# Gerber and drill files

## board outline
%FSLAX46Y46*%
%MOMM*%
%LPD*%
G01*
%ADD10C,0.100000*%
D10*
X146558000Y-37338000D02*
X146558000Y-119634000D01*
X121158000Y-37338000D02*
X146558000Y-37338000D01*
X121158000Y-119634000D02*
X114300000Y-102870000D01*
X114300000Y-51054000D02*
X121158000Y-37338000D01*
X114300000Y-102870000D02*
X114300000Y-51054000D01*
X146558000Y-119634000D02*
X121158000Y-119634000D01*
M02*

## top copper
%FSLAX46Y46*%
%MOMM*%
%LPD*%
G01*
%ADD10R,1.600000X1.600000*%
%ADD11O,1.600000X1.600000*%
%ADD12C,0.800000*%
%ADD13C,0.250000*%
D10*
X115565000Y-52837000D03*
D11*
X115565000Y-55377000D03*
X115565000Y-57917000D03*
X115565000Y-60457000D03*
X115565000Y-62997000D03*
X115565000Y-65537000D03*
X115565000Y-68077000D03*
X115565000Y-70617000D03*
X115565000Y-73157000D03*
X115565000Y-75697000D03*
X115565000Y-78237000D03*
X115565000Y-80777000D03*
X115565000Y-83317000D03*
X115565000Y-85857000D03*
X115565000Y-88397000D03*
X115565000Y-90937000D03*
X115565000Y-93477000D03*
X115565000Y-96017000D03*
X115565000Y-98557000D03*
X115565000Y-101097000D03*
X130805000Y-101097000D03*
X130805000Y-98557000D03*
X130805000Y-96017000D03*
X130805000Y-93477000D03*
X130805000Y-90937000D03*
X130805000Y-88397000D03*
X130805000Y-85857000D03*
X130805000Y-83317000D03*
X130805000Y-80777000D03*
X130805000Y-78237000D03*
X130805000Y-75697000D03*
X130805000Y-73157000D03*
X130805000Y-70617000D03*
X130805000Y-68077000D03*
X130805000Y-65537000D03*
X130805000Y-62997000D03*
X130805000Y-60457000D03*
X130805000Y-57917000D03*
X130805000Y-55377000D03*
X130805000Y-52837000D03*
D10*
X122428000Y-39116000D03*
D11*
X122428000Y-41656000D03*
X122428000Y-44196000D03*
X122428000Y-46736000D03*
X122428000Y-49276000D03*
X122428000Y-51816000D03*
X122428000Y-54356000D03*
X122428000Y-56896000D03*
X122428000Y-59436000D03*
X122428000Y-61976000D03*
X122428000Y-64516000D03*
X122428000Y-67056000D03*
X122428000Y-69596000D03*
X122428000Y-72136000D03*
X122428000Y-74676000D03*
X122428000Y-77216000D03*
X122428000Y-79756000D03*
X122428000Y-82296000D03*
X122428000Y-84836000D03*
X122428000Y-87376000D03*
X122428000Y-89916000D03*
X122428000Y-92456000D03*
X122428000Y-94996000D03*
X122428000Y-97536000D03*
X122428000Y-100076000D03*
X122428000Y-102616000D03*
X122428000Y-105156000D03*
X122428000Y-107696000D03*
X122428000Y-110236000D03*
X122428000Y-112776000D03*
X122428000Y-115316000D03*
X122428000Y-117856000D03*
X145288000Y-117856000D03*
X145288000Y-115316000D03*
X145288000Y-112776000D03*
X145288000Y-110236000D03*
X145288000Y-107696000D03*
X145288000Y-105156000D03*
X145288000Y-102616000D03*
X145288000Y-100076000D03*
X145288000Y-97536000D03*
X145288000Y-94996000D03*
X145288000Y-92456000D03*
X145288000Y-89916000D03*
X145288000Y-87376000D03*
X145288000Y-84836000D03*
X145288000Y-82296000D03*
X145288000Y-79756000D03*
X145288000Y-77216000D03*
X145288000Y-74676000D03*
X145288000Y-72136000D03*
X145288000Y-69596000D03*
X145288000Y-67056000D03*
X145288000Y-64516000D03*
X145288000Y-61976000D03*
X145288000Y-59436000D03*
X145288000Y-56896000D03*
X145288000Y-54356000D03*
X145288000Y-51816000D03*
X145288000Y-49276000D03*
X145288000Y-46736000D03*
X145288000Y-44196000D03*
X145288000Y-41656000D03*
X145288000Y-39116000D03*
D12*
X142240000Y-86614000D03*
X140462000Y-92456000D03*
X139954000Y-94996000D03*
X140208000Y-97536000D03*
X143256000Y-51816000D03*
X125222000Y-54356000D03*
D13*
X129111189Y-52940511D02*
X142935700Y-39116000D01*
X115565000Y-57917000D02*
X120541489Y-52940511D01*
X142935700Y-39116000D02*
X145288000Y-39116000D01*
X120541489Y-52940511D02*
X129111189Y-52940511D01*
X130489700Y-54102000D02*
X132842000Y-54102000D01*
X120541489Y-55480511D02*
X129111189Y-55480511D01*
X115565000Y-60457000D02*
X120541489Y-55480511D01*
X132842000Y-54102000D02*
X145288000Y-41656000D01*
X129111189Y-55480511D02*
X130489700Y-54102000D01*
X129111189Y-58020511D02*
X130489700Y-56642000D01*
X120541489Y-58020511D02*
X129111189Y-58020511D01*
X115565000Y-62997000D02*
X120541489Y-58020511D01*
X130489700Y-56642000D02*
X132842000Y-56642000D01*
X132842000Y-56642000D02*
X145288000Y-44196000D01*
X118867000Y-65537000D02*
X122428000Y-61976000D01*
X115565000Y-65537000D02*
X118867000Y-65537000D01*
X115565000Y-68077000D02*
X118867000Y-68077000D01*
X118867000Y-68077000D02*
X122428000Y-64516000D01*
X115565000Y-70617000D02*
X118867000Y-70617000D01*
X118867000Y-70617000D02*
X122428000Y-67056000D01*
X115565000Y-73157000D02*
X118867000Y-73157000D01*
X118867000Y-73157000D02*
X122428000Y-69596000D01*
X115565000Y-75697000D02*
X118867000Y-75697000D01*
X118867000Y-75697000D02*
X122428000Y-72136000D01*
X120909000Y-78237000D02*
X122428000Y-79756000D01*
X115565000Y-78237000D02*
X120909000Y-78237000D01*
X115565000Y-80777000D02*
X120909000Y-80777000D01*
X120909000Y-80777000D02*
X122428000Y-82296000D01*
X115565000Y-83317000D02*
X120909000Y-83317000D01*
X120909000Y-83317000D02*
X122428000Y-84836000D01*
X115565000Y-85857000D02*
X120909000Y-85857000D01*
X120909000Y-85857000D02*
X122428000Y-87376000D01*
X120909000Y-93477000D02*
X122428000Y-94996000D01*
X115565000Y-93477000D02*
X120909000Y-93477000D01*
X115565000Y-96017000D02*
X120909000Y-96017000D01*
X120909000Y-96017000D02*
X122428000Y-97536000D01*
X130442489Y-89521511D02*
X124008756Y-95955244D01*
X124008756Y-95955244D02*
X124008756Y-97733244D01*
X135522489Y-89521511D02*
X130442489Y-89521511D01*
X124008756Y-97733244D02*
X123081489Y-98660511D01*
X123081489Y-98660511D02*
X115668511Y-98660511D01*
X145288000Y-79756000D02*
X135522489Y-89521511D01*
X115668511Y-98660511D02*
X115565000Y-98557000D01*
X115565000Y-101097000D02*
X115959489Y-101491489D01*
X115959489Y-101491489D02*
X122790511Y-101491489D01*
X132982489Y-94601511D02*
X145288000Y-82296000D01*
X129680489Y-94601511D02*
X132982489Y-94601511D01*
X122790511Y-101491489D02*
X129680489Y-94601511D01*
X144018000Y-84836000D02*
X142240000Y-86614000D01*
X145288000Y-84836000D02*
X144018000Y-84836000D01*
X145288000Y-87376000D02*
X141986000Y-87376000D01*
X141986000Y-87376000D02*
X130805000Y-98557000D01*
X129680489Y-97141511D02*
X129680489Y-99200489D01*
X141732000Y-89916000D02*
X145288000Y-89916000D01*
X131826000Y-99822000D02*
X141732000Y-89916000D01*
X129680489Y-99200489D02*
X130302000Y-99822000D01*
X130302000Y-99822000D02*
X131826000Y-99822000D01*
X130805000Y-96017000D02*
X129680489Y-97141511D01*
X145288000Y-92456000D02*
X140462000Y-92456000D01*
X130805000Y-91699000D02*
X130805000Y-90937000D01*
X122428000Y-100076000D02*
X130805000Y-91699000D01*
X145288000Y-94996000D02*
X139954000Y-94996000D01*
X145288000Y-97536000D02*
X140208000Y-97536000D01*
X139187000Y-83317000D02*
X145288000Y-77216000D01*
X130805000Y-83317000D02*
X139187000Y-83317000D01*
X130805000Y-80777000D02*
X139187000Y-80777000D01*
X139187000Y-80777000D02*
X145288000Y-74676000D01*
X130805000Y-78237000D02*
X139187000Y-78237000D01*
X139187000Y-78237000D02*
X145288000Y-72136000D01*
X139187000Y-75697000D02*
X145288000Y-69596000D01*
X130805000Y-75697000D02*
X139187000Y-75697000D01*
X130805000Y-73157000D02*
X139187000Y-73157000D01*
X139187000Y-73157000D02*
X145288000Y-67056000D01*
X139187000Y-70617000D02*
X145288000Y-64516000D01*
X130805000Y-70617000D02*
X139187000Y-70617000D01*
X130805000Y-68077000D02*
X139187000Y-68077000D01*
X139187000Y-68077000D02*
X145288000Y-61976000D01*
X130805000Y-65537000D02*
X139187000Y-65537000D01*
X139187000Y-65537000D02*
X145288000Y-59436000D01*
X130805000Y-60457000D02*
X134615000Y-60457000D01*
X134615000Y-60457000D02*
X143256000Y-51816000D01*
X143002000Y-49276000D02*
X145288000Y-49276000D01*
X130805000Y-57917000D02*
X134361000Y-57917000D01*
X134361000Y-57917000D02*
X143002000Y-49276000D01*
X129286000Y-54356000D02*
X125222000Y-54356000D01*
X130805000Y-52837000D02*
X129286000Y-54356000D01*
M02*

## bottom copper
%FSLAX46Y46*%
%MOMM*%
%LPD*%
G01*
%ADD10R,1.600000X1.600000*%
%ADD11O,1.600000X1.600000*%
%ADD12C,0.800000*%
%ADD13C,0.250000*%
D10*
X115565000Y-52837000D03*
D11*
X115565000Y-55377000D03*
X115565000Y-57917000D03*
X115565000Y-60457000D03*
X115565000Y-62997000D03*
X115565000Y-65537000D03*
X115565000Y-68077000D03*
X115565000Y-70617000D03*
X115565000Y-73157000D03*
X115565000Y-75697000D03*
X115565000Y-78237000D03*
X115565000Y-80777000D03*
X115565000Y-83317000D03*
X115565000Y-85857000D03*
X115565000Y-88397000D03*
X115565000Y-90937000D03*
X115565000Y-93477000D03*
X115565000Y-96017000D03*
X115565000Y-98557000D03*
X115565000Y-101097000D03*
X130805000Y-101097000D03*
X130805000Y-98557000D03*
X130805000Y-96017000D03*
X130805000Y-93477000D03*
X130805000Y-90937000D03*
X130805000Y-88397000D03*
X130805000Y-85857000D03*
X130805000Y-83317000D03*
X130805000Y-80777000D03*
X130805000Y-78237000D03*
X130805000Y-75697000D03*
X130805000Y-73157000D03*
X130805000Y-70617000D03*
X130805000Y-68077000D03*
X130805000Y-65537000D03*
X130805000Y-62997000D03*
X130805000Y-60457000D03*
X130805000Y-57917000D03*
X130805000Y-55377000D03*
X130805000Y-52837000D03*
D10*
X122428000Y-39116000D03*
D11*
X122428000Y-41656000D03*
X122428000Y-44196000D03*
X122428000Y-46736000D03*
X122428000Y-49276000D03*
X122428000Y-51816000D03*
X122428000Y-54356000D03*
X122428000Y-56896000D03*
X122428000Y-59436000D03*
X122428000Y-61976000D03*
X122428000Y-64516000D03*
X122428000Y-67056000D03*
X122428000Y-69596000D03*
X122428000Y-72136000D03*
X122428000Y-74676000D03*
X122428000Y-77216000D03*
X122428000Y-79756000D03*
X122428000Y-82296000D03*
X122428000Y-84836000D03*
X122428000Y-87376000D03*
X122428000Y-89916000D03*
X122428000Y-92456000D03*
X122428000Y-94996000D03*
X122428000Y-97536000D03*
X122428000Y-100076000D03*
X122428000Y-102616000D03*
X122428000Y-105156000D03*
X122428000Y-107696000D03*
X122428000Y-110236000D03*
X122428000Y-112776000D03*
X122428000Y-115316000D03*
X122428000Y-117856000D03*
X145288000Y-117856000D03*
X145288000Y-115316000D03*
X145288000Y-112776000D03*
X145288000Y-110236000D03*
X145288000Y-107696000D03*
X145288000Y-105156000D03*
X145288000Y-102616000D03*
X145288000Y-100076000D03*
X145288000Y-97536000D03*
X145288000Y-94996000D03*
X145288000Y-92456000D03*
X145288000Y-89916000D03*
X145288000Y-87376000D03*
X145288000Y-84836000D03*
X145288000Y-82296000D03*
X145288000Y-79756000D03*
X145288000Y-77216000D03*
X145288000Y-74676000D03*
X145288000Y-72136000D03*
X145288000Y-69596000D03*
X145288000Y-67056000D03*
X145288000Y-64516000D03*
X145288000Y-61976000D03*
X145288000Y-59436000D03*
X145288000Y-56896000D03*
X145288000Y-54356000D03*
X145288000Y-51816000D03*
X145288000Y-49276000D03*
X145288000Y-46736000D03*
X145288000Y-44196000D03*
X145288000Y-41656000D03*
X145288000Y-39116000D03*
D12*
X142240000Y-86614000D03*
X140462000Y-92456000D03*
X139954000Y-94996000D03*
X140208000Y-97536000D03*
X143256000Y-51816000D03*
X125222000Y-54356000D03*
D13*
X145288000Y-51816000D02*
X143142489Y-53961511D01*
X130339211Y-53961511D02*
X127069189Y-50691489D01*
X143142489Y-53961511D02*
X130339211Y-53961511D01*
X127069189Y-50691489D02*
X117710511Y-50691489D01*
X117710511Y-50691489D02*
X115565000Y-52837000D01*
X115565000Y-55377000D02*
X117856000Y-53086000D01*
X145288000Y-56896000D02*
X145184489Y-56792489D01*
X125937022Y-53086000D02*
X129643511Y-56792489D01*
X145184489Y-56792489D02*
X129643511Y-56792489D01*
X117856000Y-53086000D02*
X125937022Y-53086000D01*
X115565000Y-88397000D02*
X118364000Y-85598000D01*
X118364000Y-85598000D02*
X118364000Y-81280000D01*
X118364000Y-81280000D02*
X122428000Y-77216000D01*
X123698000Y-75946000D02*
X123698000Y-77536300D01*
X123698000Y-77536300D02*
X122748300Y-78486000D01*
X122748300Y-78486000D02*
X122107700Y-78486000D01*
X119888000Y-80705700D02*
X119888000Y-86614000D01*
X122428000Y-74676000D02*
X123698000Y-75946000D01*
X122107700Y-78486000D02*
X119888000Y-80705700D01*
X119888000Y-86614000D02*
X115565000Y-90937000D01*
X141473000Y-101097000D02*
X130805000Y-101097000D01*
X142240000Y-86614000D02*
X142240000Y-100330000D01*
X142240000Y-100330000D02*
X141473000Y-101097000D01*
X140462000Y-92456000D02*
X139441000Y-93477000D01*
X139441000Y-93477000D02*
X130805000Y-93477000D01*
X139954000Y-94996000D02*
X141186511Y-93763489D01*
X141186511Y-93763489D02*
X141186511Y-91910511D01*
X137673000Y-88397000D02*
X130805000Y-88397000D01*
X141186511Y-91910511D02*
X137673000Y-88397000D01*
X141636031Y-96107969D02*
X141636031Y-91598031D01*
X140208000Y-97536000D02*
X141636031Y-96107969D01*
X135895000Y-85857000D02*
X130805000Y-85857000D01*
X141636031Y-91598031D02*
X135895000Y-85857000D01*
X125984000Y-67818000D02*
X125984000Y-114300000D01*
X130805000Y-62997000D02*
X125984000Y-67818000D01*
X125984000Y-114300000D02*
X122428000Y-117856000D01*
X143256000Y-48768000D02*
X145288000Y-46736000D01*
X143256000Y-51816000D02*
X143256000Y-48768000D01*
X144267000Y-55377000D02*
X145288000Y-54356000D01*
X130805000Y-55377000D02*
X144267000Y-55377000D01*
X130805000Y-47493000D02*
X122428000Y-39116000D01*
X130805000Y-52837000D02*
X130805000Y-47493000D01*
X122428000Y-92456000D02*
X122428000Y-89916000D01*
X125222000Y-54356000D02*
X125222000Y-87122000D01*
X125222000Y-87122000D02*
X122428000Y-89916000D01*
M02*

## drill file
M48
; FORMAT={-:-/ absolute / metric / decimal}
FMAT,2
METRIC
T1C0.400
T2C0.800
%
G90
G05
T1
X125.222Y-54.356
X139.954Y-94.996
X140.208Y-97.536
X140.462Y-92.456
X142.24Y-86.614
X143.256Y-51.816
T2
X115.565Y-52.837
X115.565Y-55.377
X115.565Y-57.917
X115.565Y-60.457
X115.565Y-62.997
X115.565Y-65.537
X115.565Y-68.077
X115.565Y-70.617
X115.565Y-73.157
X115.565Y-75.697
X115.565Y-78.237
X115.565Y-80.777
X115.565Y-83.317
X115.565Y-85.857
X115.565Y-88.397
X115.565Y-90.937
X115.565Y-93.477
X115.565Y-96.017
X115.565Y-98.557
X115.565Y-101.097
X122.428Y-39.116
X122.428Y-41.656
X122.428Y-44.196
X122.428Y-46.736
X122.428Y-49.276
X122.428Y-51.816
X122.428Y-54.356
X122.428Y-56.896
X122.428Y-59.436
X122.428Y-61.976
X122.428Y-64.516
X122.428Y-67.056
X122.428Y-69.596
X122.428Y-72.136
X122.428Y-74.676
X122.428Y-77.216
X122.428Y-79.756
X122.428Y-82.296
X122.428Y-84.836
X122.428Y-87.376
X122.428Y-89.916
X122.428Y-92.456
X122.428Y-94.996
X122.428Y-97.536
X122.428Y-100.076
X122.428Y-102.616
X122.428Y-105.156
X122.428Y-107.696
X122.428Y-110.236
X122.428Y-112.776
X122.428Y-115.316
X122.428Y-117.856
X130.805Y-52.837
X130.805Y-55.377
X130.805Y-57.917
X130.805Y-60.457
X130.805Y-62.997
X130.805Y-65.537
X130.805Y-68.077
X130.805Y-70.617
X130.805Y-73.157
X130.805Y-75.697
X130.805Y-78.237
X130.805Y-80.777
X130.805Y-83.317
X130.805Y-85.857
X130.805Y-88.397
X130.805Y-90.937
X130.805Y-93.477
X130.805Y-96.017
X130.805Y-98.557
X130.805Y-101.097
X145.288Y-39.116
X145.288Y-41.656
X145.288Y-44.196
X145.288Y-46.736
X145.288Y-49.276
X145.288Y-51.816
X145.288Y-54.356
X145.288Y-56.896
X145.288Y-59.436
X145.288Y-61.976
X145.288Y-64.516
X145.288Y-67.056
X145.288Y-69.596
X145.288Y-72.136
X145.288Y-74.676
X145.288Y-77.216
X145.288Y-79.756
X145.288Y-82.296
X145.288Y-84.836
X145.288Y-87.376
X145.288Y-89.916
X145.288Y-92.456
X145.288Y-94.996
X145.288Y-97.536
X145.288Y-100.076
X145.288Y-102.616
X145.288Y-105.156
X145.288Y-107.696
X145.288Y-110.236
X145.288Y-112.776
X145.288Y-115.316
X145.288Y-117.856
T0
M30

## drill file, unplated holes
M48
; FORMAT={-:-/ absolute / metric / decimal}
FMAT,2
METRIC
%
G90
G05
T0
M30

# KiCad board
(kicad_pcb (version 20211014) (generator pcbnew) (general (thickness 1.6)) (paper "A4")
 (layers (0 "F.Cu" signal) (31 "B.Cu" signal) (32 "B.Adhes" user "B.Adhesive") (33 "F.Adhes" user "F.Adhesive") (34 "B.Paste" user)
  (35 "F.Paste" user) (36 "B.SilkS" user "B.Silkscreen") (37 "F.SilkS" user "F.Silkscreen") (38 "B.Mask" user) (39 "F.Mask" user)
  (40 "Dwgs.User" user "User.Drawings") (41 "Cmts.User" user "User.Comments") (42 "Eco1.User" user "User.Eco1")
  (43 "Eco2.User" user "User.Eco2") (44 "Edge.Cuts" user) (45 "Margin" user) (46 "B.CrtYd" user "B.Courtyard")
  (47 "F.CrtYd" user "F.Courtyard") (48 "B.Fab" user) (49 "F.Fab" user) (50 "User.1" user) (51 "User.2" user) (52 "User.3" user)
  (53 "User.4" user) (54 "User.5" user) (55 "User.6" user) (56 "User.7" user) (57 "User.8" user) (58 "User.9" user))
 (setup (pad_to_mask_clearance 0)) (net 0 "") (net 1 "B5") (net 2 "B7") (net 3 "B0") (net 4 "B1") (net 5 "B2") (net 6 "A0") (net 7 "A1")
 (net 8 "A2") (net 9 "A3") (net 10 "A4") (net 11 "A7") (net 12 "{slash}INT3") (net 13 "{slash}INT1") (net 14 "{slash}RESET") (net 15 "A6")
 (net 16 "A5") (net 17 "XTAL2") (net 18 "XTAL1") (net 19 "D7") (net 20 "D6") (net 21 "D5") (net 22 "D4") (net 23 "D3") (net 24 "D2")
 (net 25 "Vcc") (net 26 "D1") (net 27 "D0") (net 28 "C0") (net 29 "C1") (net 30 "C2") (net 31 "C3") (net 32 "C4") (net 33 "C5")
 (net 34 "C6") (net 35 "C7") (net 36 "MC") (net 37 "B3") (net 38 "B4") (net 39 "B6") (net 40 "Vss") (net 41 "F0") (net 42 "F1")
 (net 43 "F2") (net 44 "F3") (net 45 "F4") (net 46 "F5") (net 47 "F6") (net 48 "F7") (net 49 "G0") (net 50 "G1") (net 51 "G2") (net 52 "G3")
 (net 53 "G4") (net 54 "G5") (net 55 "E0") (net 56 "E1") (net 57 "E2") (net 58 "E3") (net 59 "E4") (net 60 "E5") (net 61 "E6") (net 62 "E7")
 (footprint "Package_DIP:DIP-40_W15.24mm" (layer "F.Cu") (at 115.565 52.837)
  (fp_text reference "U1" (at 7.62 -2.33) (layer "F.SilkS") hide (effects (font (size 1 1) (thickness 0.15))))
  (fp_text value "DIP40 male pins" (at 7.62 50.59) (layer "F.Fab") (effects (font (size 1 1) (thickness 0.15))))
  (pad "1" thru_hole rect locked (at 0 0) (size 1.6 1.6) (drill 0.8) (layers *.Cu *.Mask) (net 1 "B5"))
  (pad "2" thru_hole oval locked (at 0 2.54) (size 1.6 1.6) (drill 0.8) (layers *.Cu *.Mask) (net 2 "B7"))
  (pad "3" thru_hole oval locked (at 0 5.08) (size 1.6 1.6) (drill 0.8) (layers *.Cu *.Mask) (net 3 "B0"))
  (pad "4" thru_hole oval locked (at 0 7.62) (size 1.6 1.6) (drill 0.8) (layers *.Cu *.Mask) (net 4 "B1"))
  (pad "5" thru_hole oval locked (at 0 10.16) (size 1.6 1.6) (drill 0.8) (layers *.Cu *.Mask) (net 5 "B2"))
  (pad "6" thru_hole oval locked (at 0 12.7) (size 1.6 1.6) (drill 0.8) (layers *.Cu *.Mask) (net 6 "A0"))
  (pad "7" thru_hole oval locked (at 0 15.24) (size 1.6 1.6) (drill 0.8) (layers *.Cu *.Mask) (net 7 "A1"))
  (pad "8" thru_hole oval locked (at 0 17.78) (size 1.6 1.6) (drill 0.8) (layers *.Cu *.Mask) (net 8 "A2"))
  (pad "9" thru_hole oval locked (at 0 20.32) (size 1.6 1.6) (drill 0.8) (layers *.Cu *.Mask) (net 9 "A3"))
  (pad "10" thru_hole oval locked (at 0 22.86) (size 1.6 1.6) (drill 0.8) (layers *.Cu *.Mask) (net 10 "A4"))
  (pad "11" thru_hole oval locked (at 0 25.4) (size 1.6 1.6) (drill 0.8) (layers *.Cu *.Mask) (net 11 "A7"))
  (pad "12" thru_hole oval locked (at 0 27.94) (size 1.6 1.6) (drill 0.8) (layers *.Cu *.Mask) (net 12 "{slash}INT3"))
  (pad "13" thru_hole oval locked (at 0 30.48) (size 1.6 1.6) (drill 0.8) (layers *.Cu *.Mask) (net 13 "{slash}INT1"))
  (pad "14" thru_hole oval locked (at 0 33.02) (size 1.6 1.6) (drill 0.8) (layers *.Cu *.Mask) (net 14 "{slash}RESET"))
  (pad "15" thru_hole oval locked (at 0 35.56) (size 1.6 1.6) (drill 0.8) (layers *.Cu *.Mask) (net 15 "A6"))
  (pad "16" thru_hole oval locked (at 0 38.1) (size 1.6 1.6) (drill 0.8) (layers *.Cu *.Mask) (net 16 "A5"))
  (pad "17" thru_hole oval locked (at 0 40.64) (size 1.6 1.6) (drill 0.8) (layers *.Cu *.Mask) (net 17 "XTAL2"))
  (pad "18" thru_hole oval locked (at 0 43.18) (size 1.6 1.6) (drill 0.8) (layers *.Cu *.Mask) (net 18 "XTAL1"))
  (pad "19" thru_hole oval locked (at 0 45.72) (size 1.6 1.6) (drill 0.8) (layers *.Cu *.Mask) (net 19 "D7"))
  (pad "20" thru_hole oval locked (at 0 48.26) (size 1.6 1.6) (drill 0.8) (layers *.Cu *.Mask) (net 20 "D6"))
  (pad "21" thru_hole oval locked (at 15.24 48.26) (size 1.6 1.6) (drill 0.8) (layers *.Cu *.Mask) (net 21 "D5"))
  (pad "22" thru_hole oval locked (at 15.24 45.72) (size 1.6 1.6) (drill 0.8) (layers *.Cu *.Mask) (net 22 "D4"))
  (pad "23" thru_hole oval locked (at 15.24 43.18) (size 1.6 1.6) (drill 0.8) (layers *.Cu *.Mask) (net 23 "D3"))
  (pad "24" thru_hole oval locked (at 15.24 40.64) (size 1.6 1.6) (drill 0.8) (layers *.Cu *.Mask) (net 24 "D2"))
  (pad "25" thru_hole oval locked (at 15.24 38.1) (size 1.6 1.6) (drill 0.8) (layers *.Cu *.Mask) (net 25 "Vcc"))
  (pad "26" thru_hole oval locked (at 15.24 35.56) (size 1.6 1.6) (drill 0.8) (layers *.Cu *.Mask) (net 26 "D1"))
  (pad "27" thru_hole oval locked (at 15.24 33.02) (size 1.6 1.6) (drill 0.8) (layers *.Cu *.Mask) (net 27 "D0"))
  (pad "28" thru_hole oval locked (at 15.24 30.48) (size 1.6 1.6) (drill 0.8) (layers *.Cu *.Mask) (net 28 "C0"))
  (pad "29" thru_hole oval locked (at 15.24 27.94) (size 1.6 1.6) (drill 0.8) (layers *.Cu *.Mask) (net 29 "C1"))
  (pad "30" thru_hole oval locked (at 15.24 25.4) (size 1.6 1.6) (drill 0.8) (layers *.Cu *.Mask) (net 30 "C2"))
  (pad "31" thru_hole oval locked (at 15.24 22.86) (size 1.6 1.6) (drill 0.8) (layers *.Cu *.Mask) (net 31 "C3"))
  (pad "32" thru_hole oval locked (at 15.24 20.32) (size 1.6 1.6) (drill 0.8) (layers *.Cu *.Mask) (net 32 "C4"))
  (pad "33" thru_hole oval locked (at 15.24 17.78) (size 1.6 1.6) (drill 0.8) (layers *.Cu *.Mask) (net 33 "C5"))
  (pad "34" thru_hole oval locked (at 15.24 15.24) (size 1.6 1.6) (drill 0.8) (layers *.Cu *.Mask) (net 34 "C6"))
  (pad "35" thru_hole oval locked (at 15.24 12.7) (size 1.6 1.6) (drill 0.8) (layers *.Cu *.Mask) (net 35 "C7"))
  (pad "36" thru_hole oval locked (at 15.24 10.16) (size 1.6 1.6) (drill 0.8) (layers *.Cu *.Mask) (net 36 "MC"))
  (pad "37" thru_hole oval locked (at 15.24 7.62) (size 1.6 1.6) (drill 0.8) (layers *.Cu *.Mask) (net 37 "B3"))
  (pad "38" thru_hole oval locked (at 15.24 5.08) (size 1.6 1.6) (drill 0.8) (layers *.Cu *.Mask) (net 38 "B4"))
  (pad "39" thru_hole oval locked (at 15.24 2.54) (size 1.6 1.6) (drill 0.8) (layers *.Cu *.Mask) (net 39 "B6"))
  (pad "40" thru_hole oval locked (at 15.24 0) (size 1.6 1.6) (drill 0.8) (layers *.Cu *.Mask) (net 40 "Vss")))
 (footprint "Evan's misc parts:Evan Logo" (layer "F.Cu") (at 118.11 105.156)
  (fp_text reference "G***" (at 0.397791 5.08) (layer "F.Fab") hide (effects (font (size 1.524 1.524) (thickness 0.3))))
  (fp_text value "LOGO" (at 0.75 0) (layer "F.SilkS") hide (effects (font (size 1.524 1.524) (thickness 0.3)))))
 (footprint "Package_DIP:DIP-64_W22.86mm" (layer "F.Cu") (at 122.428 39.116)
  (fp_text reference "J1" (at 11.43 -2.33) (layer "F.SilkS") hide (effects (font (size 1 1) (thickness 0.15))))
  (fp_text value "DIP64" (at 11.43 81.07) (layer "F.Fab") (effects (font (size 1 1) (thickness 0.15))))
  (pad "1" thru_hole rect locked (at 0 0) (size 1.6 1.6) (drill 0.8) (layers *.Cu *.Mask) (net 40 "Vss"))
  (pad "2" thru_hole oval locked (at 0 2.54) (size 1.6 1.6) (drill 0.8) (layers *.Cu *.Mask) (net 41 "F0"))
  (pad "3" thru_hole oval locked (at 0 5.08) (size 1.6 1.6) (drill 0.8) (layers *.Cu *.Mask) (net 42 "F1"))
  (pad "4" thru_hole oval locked (at 0 7.62) (size 1.6 1.6) (drill 0.8) (layers *.Cu *.Mask) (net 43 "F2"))
  (pad "5" thru_hole oval locked (at 0 10.16) (size 1.6 1.6) (drill 0.8) (layers *.Cu *.Mask) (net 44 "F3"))
  (pad "6" thru_hole oval locked (at 0 12.7) (size 1.6 1.6) (drill 0.8) (layers *.Cu *.Mask) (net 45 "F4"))
  (pad "7" thru_hole oval locked (at 0 15.24) (size 1.6 1.6) (drill 0.8) (layers *.Cu *.Mask) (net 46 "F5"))
  (pad "8" thru_hole oval locked (at 0 17.78) (size 1.6 1.6) (drill 0.8) (layers *.Cu *.Mask) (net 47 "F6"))
  (pad "9" thru_hole oval locked (at 0 20.32) (size 1.6 1.6) (drill 0.8) (layers *.Cu *.Mask) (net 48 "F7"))
  (pad "10" thru_hole oval locked (at 0 22.86) (size 1.6 1.6) (drill 0.8) (layers *.Cu *.Mask) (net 6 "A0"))
  (pad "11" thru_hole oval locked (at 0 25.4) (size 1.6 1.6) (drill 0.8) (layers *.Cu *.Mask) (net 7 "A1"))
  (pad "12" thru_hole oval locked (at 0 27.94) (size 1.6 1.6) (drill 0.8) (layers *.Cu *.Mask) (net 8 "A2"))
  (pad "13" thru_hole oval locked (at 0 30.48) (size 1.6 1.6) (drill 0.8) (layers *.Cu *.Mask) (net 9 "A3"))
  (pad "14" thru_hole oval locked (at 0 33.02) (size 1.6 1.6) (drill 0.8) (layers *.Cu *.Mask) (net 10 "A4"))
  (pad "15" thru_hole oval locked (at 0 35.56) (size 1.6 1.6) (drill 0.8) (layers *.Cu *.Mask) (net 16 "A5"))
  (pad "16" thru_hole oval locked (at 0 38.1) (size 1.6 1.6) (drill 0.8) (layers *.Cu *.Mask) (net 15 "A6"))
  (pad "17" thru_hole oval locked (at 0 40.64) (size 1.6 1.6) (drill 0.8) (layers *.Cu *.Mask) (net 11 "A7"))
  (pad "18" thru_hole oval locked (at 0 43.18) (size 1.6 1.6) (drill 0.8) (layers *.Cu *.Mask) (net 12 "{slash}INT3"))
  (pad "19" thru_hole oval locked (at 0 45.72) (size 1.6 1.6) (drill 0.8) (layers *.Cu *.Mask) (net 13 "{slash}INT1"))
  (pad "20" thru_hole oval locked (at 0 48.26) (size 1.6 1.6) (drill 0.8) (layers *.Cu *.Mask) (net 14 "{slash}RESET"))
  (pad "21" thru_hole oval locked (at 0 50.8) (size 1.6 1.6) (drill 0.8) (layers *.Cu *.Mask) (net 40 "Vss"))
  (pad "22" thru_hole oval locked (at 0 53.34) (size 1.6 1.6) (drill 0.8) (layers *.Cu *.Mask) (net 40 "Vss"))
  (pad "23" thru_hole oval locked (at 0 55.88) (size 1.6 1.6) (drill 0.8) (layers *.Cu *.Mask) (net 17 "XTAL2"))
  (pad "24" thru_hole oval locked (at 0 58.42) (size 1.6 1.6) (drill 0.8) (layers *.Cu *.Mask) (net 18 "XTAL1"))
  (pad "25" thru_hole oval locked (at 0 60.96) (size 1.6 1.6) (drill 0.8) (layers *.Cu *.Mask) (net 25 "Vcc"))
  (pad "26" thru_hole oval locked (at 0 63.5) (size 1.6 1.6) (drill 0.8) (layers *.Cu *.Mask) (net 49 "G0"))
  (pad "27" thru_hole oval locked (at 0 66.04) (size 1.6 1.6) (drill 0.8) (layers *.Cu *.Mask) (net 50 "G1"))
  (pad "28" thru_hole oval locked (at 0 68.58) (size 1.6 1.6) (drill 0.8) (layers *.Cu *.Mask) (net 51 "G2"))
  (pad "29" thru_hole oval locked (at 0 71.12) (size 1.6 1.6) (drill 0.8) (layers *.Cu *.Mask) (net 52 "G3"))
  (pad "30" thru_hole oval locked (at 0 73.66) (size 1.6 1.6) (drill 0.8) (layers *.Cu *.Mask) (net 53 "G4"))
  (pad "31" thru_hole oval locked (at 0 76.2) (size 1.6 1.6) (drill 0.8) (layers *.Cu *.Mask) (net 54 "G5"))
  (pad "32" thru_hole oval locked (at 0 78.74) (size 1.6 1.6) (drill 0.8) (layers *.Cu *.Mask) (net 36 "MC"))
  (pad "33" thru_hole oval locked (at 22.86 78.74) (size 1.6 1.6) (drill 0.8) (layers *.Cu *.Mask) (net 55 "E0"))
  (pad "34" thru_hole oval locked (at 22.86 76.2) (size 1.6 1.6) (drill 0.8) (layers *.Cu *.Mask) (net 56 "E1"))
  (pad "35" thru_hole oval locked (at 22.86 73.66) (size 1.6 1.6) (drill 0.8) (layers *.Cu *.Mask) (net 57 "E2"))
  (pad "36" thru_hole oval locked (at 22.86 71.12) (size 1.6 1.6) (drill 0.8) (layers *.Cu *.Mask) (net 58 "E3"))
  (pad "37" thru_hole oval locked (at 22.86 68.58) (size 1.6 1.6) (drill 0.8) (layers *.Cu *.Mask) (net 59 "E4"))
  (pad "38" thru_hole oval locked (at 22.86 66.04) (size 1.6 1.6) (drill 0.8) (layers *.Cu *.Mask) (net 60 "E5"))
  (pad "39" thru_hole oval locked (at 22.86 63.5) (size 1.6 1.6) (drill 0.8) (layers *.Cu *.Mask) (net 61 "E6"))
  (pad "40" thru_hole oval locked (at 22.86 60.96) (size 1.6 1.6) (drill 0.8) (layers *.Cu *.Mask) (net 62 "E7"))
  (pad "41" thru_hole oval locked (at 22.86 58.42) (size 1.6 1.6) (drill 0.8) (layers *.Cu *.Mask) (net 27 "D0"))
  (pad "42" thru_hole oval locked (at 22.86 55.88) (size 1.6 1.6) (drill 0.8) (layers *.Cu *.Mask) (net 26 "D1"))
  (pad "43" thru_hole oval locked (at 22.86 53.34) (size 1.6 1.6) (drill 0.8) (layers *.Cu *.Mask) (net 24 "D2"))
  (pad "44" thru_hole oval locked (at 22.86 50.8) (size 1.6 1.6) (drill 0.8) (layers *.Cu *.Mask) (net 23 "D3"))
  (pad "45" thru_hole oval locked (at 22.86 48.26) (size 1.6 1.6) (drill 0.8) (layers *.Cu *.Mask) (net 22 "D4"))
  (pad "46" thru_hole oval locked (at 22.86 45.72) (size 1.6 1.6) (drill 0.8) (layers *.Cu *.Mask) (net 21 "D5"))
  (pad "47" thru_hole oval locked (at 22.86 43.18) (size 1.6 1.6) (drill 0.8) (layers *.Cu *.Mask) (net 20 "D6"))
  (pad "48" thru_hole oval locked (at 22.86 40.64) (size 1.6 1.6) (drill 0.8) (layers *.Cu *.Mask) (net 19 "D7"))
  (pad "49" thru_hole oval locked (at 22.86 38.1) (size 1.6 1.6) (drill 0.8) (layers *.Cu *.Mask) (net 28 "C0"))
  (pad "50" thru_hole oval locked (at 22.86 35.56) (size 1.6 1.6) (drill 0.8) (layers *.Cu *.Mask) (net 29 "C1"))
  (pad "51" thru_hole oval locked (at 22.86 33.02) (size 1.6 1.6) (drill 0.8) (layers *.Cu *.Mask) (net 30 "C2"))
  (pad "52" thru_hole oval locked (at 22.86 30.48) (size 1.6 1.6) (drill 0.8) (layers *.Cu *.Mask) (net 31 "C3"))
  (pad "53" thru_hole oval locked (at 22.86 27.94) (size 1.6 1.6) (drill 0.8) (layers *.Cu *.Mask) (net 32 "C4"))
  (pad "54" thru_hole oval locked (at 22.86 25.4) (size 1.6 1.6) (drill 0.8) (layers *.Cu *.Mask) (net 33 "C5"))
  (pad "55" thru_hole oval locked (at 22.86 22.86) (size 1.6 1.6) (drill 0.8) (layers *.Cu *.Mask) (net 34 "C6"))
  (pad "56" thru_hole oval locked (at 22.86 20.32) (size 1.6 1.6) (drill 0.8) (layers *.Cu *.Mask) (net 35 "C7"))
  (pad "57" thru_hole oval locked (at 22.86 17.78) (size 1.6 1.6) (drill 0.8) (layers *.Cu *.Mask) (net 2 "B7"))
  (pad "58" thru_hole oval locked (at 22.86 15.24) (size 1.6 1.6) (drill 0.8) (layers *.Cu *.Mask) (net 39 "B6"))
  (pad "59" thru_hole oval locked (at 22.86 12.7) (size 1.6 1.6) (drill 0.8) (layers *.Cu *.Mask) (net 1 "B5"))
  (pad "60" thru_hole oval locked (at 22.86 10.16) (size 1.6 1.6) (drill 0.8) (layers *.Cu *.Mask) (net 38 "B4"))
  (pad "61" thru_hole oval locked (at 22.86 7.62) (size 1.6 1.6) (drill 0.8) (layers *.Cu *.Mask) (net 37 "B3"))
  (pad "62" thru_hole oval locked (at 22.86 5.08) (size 1.6 1.6) (drill 0.8) (layers *.Cu *.Mask) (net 5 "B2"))
  (pad "63" thru_hole oval locked (at 22.86 2.54) (size 1.6 1.6) (drill 0.8) (layers *.Cu *.Mask) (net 4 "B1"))
  (pad "64" thru_hole oval locked (at 22.86 0) (size 1.6 1.6) (drill 0.8) (layers *.Cu *.Mask) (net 3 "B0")))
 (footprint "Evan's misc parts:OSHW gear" (layer "B.Cu") (at 118.364 104.902 180)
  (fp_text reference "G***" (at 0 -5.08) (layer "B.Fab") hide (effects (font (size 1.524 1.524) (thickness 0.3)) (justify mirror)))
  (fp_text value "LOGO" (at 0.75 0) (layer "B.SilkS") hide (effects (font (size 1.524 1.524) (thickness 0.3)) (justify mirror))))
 (gr_line (start 146.558 37.338) (end 146.558 119.634) (layer "Edge.Cuts") (width 0.1))
 (gr_line (start 121.158 37.338) (end 146.558 37.338) (layer "Edge.Cuts") (width 0.1))
 (gr_line (start 121.158 119.634) (end 114.3 102.87) (layer "Edge.Cuts") (width 0.1))
 (gr_line (start 114.3 51.054) (end 121.158 37.338) (layer "Edge.Cuts") (width 0.1))
 (gr_line (start 114.3 102.87) (end 114.3 51.054) (layer "Edge.Cuts") (width 0.1))
 (gr_line (start 146.558 119.634) (end 121.158 119.634) (layer "Edge.Cuts") (width 0.1))
 (segment (start 145.288 51.816) (end 143.142489 53.961511) (width 0.25) (layer "B.Cu") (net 1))
 (segment (start 130.339211 53.961511) (end 127.069189 50.691489) (width 0.25) (layer "B.Cu") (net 1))
 (segment (start 143.142489 53.961511) (end 130.339211 53.961511) (width 0.25) (layer "B.Cu") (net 1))
 (segment (start 127.069189 50.691489) (end 117.710511 50.691489) (width 0.25) (layer "B.Cu") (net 1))
 (segment (start 117.710511 50.691489) (end 115.565 52.837) (width 0.25) (layer "B.Cu") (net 1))
 (segment (start 115.565 55.377) (end 117.856 53.086) (width 0.25) (layer "B.Cu") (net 2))
 (segment (start 145.288 56.896) (end 145.184489 56.792489) (width 0.25) (layer "B.Cu") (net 2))
 (segment (start 125.937022 53.086) (end 129.643511 56.792489) (width 0.25) (layer "B.Cu") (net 2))
 (segment (start 145.184489 56.792489) (end 129.643511 56.792489) (width 0.25) (layer "B.Cu") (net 2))
 (segment (start 117.856 53.086) (end 125.937022 53.086) (width 0.25) (layer "B.Cu") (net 2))
 (segment (start 129.111189 52.940511) (end 142.9357 39.116) (width 0.25) (layer "F.Cu") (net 3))
 (segment (start 115.565 57.917) (end 120.541489 52.940511) (width 0.25) (layer "F.Cu") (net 3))
 (segment (start 142.9357 39.116) (end 145.288 39.116) (width 0.25) (layer "F.Cu") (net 3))
 (segment (start 120.541489 52.940511) (end 129.111189 52.940511) (width 0.25) (layer "F.Cu") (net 3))
 (segment (start 130.4897 54.102) (end 132.842 54.102) (width 0.25) (layer "F.Cu") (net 4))
 (segment (start 120.541489 55.480511) (end 129.111189 55.480511) (width 0.25) (layer "F.Cu") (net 4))
 (segment (start 115.565 60.457) (end 120.541489 55.480511) (width 0.25) (layer "F.Cu") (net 4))
 (segment (start 132.842 54.102) (end 145.288 41.656) (width 0.25) (layer "F.Cu") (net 4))
 (segment (start 129.111189 55.480511) (end 130.4897 54.102) (width 0.25) (layer "F.Cu") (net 4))
 (segment (start 129.111189 58.020511) (end 130.4897 56.642) (width 0.25) (layer "F.Cu") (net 5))
 (segment (start 120.541489 58.020511) (end 129.111189 58.020511) (width 0.25) (layer "F.Cu") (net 5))
 (segment (start 115.565 62.997) (end 120.541489 58.020511) (width 0.25) (layer "F.Cu") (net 5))
 (segment (start 130.4897 56.642) (end 132.842 56.642) (width 0.25) (layer "F.Cu") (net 5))
 (segment (start 132.842 56.642) (end 145.288 44.196) (width 0.25) (layer "F.Cu") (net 5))
 (segment (start 118.867 65.537) (end 122.428 61.976) (width 0.25) (layer "F.Cu") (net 6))
 (segment (start 115.565 65.537) (end 118.867 65.537) (width 0.25) (layer "F.Cu") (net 6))
 (segment (start 115.565 68.077) (end 118.867 68.077) (width 0.25) (layer "F.Cu") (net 7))
 (segment (start 118.867 68.077) (end 122.428 64.516) (width 0.25) (layer "F.Cu") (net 7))
 (segment (start 115.565 70.617) (end 118.867 70.617) (width 0.25) (layer "F.Cu") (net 8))
 (segment (start 118.867 70.617) (end 122.428 67.056) (width 0.25) (layer "F.Cu") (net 8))
 (segment (start 115.565 73.157) (end 118.867 73.157) (width 0.25) (layer "F.Cu") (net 9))
 (segment (start 118.867 73.157) (end 122.428 69.596) (width 0.25) (layer "F.Cu") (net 9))
 (segment (start 115.565 75.697) (end 118.867 75.697) (width 0.25) (layer "F.Cu") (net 10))
 (segment (start 118.867 75.697) (end 122.428 72.136) (width 0.25) (layer "F.Cu") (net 10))
 (segment (start 120.909 78.237) (end 122.428 79.756) (width 0.25) (layer "F.Cu") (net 11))
 (segment (start 115.565 78.237) (end 120.909 78.237) (width 0.25) (layer "F.Cu") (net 11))
 (segment (start 115.565 80.777) (end 120.909 80.777) (width 0.25) (layer "F.Cu") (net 12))
 (segment (start 120.909 80.777) (end 122.428 82.296) (width 0.25) (layer "F.Cu") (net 12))
 (segment (start 115.565 83.317) (end 120.909 83.317) (width 0.25) (layer "F.Cu") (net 13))
 (segment (start 120.909 83.317) (end 122.428 84.836) (width 0.25) (layer "F.Cu") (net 13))
 (segment (start 115.565 85.857) (end 120.909 85.857) (width 0.25) (layer "F.Cu") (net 14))
 (segment (start 120.909 85.857) (end 122.428 87.376) (width 0.25) (layer "F.Cu") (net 14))
 (segment (start 115.565 88.397) (end 118.364 85.598) (width 0.25) (layer "B.Cu") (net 15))
 (segment (start 118.364 85.598) (end 118.364 81.28) (width 0.25) (layer "B.Cu") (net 15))
 (segment (start 118.364 81.28) (end 122.428 77.216) (width 0.25) (layer "B.Cu") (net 15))
 (segment (start 123.698 75.946) (end 123.698 77.5363) (width 0.25) (layer "B.Cu") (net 16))
 (segment (start 123.698 77.5363) (end 122.7483 78.486) (width 0.25) (layer "B.Cu") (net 16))
 (segment (start 122.7483 78.486) (end 122.1077 78.486) (width 0.25) (layer "B.Cu") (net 16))
 (segment (start 119.888 80.7057) (end 119.888 86.614) (width 0.25) (layer "B.Cu") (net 16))
 (segment (start 122.428 74.676) (end 123.698 75.946) (width 0.25) (layer "B.Cu") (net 16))
 (segment (start 122.1077 78.486) (end 119.888 80.7057) (width 0.25) (layer "B.Cu") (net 16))
 (segment (start 119.888 86.614) (end 115.565 90.937) (width 0.25) (layer "B.Cu") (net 16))
 (segment (start 120.909 93.477) (end 122.428 94.996) (width 0.25) (layer "F.Cu") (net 17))
 (segment (start 115.565 93.477) (end 120.909 93.477) (width 0.25) (layer "F.Cu") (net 17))
 (segment (start 115.565 96.017) (end 120.909 96.017) (width 0.25) (layer "F.Cu") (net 18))
 (segment (start 120.909 96.017) (end 122.428 97.536) (width 0.25) (layer "F.Cu") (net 18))
 (segment (start 130.442489 89.521511) (end 124.008756 95.955244) (width 0.25) (layer "F.Cu") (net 19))
 (segment (start 124.008756 95.955244) (end 124.008756 97.733244) (width 0.25) (layer "F.Cu") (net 19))
 (segment (start 135.522489 89.521511) (end 130.442489 89.521511) (width 0.25) (layer "F.Cu") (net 19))
 (segment (start 124.008756 97.733244) (end 123.081489 98.660511) (width 0.25) (layer "F.Cu") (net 19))
 (segment (start 123.081489 98.660511) (end 115.668511 98.660511) (width 0.25) (layer "F.Cu") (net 19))
 (segment (start 145.288 79.756) (end 135.522489 89.521511) (width 0.25) (layer "F.Cu") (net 19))
 (segment (start 115.668511 98.660511) (end 115.565 98.557) (width 0.25) (layer "F.Cu") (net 19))
 (segment (start 115.565 101.097) (end 115.959489 101.491489) (width 0.25) (layer "F.Cu") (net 20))
 (segment (start 115.959489 101.491489) (end 122.790511 101.491489) (width 0.25) (layer "F.Cu") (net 20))
 (segment (start 132.982489 94.601511) (end 145.288 82.296) (width 0.25) (layer "F.Cu") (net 20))
 (segment (start 129.680489 94.601511) (end 132.982489 94.601511) (width 0.25) (layer "F.Cu") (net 20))
 (segment (start 122.790511 101.491489) (end 129.680489 94.601511) (width 0.25) (layer "F.Cu") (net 20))
 (segment (start 144.018 84.836) (end 142.24 86.614) (width 0.25) (layer "F.Cu") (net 21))
 (segment (start 145.288 84.836) (end 144.018 84.836) (width 0.25) (layer "F.Cu") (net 21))
 (via (at 142.24 86.614) (size 0.8) (drill 0.4) (layers "F.Cu" "B.Cu") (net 21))
 (segment (start 141.473 101.097) (end 130.805 101.097) (width 0.25) (layer "B.Cu") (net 21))
 (segment (start 142.24 86.614) (end 142.24 100.33) (width 0.25) (layer "B.Cu") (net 21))
 (segment (start 142.24 100.33) (end 141.473 101.097) (width 0.25) (layer "B.Cu") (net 21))
 (segment (start 145.288 87.376) (end 141.986 87.376) (width 0.25) (layer "F.Cu") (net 22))
 (segment (start 141.986 87.376) (end 130.805 98.557) (width 0.25) (layer "F.Cu") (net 22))
 (segment (start 129.680489 97.141511) (end 129.680489 99.200489) (width 0.25) (layer "F.Cu") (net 23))
 (segment (start 141.732 89.916) (end 145.288 89.916) (width 0.25) (layer "F.Cu") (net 23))
 (segment (start 131.826 99.822) (end 141.732 89.916) (width 0.25) (layer "F.Cu") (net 23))
 (segment (start 129.680489 99.200489) (end 130.302 99.822) (width 0.25) (layer "F.Cu") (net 23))
 (segment (start 130.302 99.822) (end 131.826 99.822) (width 0.25) (layer "F.Cu") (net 23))
 (segment (start 130.805 96.017) (end 129.680489 97.141511) (width 0.25) (layer "F.Cu") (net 23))
 (segment (start 145.288 92.456) (end 140.462 92.456) (width 0.25) (layer "F.Cu") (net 24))
 (via (at 140.462 92.456) (size 0.8) (drill 0.4) (layers "F.Cu" "B.Cu") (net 24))
 (segment (start 140.462 92.456) (end 139.441 93.477) (width 0.25) (layer "B.Cu") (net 24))
 (segment (start 139.441 93.477) (end 130.805 93.477) (width 0.25) (layer "B.Cu") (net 24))
 (segment (start 130.805 91.699) (end 130.805 90.937) (width 0.25) (layer "F.Cu") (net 25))
 (segment (start 122.428 100.076) (end 130.805 91.699) (width 0.25) (layer "F.Cu") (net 25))
 (segment (start 145.288 94.996) (end 139.954 94.996) (width 0.25) (layer "F.Cu") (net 26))
 (via (at 139.954 94.996) (size 0.8) (drill 0.4) (layers "F.Cu" "B.Cu") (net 26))
 (segment (start 139.954 94.996) (end 141.186511 93.763489) (width 0.25) (layer "B.Cu") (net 26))
 (segment (start 141.186511 93.763489) (end 141.186511 91.910511) (width 0.25) (layer "B.Cu") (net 26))
 (segment (start 137.673 88.397) (end 130.805 88.397) (width 0.25) (layer "B.Cu") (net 26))
 (segment (start 141.186511 91.910511) (end 137.673 88.397) (width 0.25) (layer "B.Cu") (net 26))
 (segment (start 145.288 97.536) (end 140.208 97.536) (width 0.25) (layer "F.Cu") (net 27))
 (via (at 140.208 97.536) (size 0.8) (drill 0.4) (layers "F.Cu" "B.Cu") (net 27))
 (segment (start 141.636031 96.107969) (end 141.636031 91.598031) (width 0.25) (layer "B.Cu") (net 27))
 (segment (start 140.208 97.536) (end 141.636031 96.107969) (width 0.25) (layer "B.Cu") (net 27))
 (segment (start 135.895 85.857) (end 130.805 85.857) (width 0.25) (layer "B.Cu") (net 27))
 (segment (start 141.636031 91.598031) (end 135.895 85.857) (width 0.25) (layer "B.Cu") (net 27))
 (segment (start 139.187 83.317) (end 145.288 77.216) (width 0.25) (layer "F.Cu") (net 28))
 (segment (start 130.805 83.317) (end 139.187 83.317) (width 0.25) (layer "F.Cu") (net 28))
 (segment (start 130.805 80.777) (end 139.187 80.777) (width 0.25) (layer "F.Cu") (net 29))
 (segment (start 139.187 80.777) (end 145.288 74.676) (width 0.25) (layer "F.Cu") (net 29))
 (segment (start 130.805 78.237) (end 139.187 78.237) (width 0.25) (layer "F.Cu") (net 30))
 (segment (start 139.187 78.237) (end 145.288 72.136) (width 0.25) (layer "F.Cu") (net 30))
 (segment (start 139.187 75.697) (end 145.288 69.596) (width 0.25) (layer "F.Cu") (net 31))
 (segment (start 130.805 75.697) (end 139.187 75.697) (width 0.25) (layer "F.Cu") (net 31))
 (segment (start 130.805 73.157) (end 139.187 73.157) (width 0.25) (layer "F.Cu") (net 32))
 (segment (start 139.187 73.157) (end 145.288 67.056) (width 0.25) (layer "F.Cu") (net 32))
 (segment (start 139.187 70.617) (end 145.288 64.516) (width 0.25) (layer "F.Cu") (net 33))
 (segment (start 130.805 70.617) (end 139.187 70.617) (width 0.25) (layer "F.Cu") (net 33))
 (segment (start 130.805 68.077) (end 139.187 68.077) (width 0.25) (layer "F.Cu") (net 34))
 (segment (start 139.187 68.077) (end 145.288 61.976) (width 0.25) (layer "F.Cu") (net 34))
 (segment (start 130.805 65.537) (end 139.187 65.537) (width 0.25) (layer "F.Cu") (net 35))
 (segment (start 139.187 65.537) (end 145.288 59.436) (width 0.25) (layer "F.Cu") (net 35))
 (segment (start 125.984 67.818) (end 125.984 114.3) (width 0.25) (layer "B.Cu") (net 36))
 (segment (start 130.805 62.997) (end 125.984 67.818) (width 0.25) (layer "B.Cu") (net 36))
 (segment (start 125.984 114.3) (end 122.428 117.856) (width 0.25) (layer "B.Cu") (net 36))
 (segment (start 130.805 60.457) (end 134.615 60.457) (width 0.25) (layer "F.Cu") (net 37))
 (segment (start 134.615 60.457) (end 143.256 51.816) (width 0.25) (layer "F.Cu") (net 37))
 (via (at 143.256 51.816) (size 0.8) (drill 0.4) (layers "F.Cu" "B.Cu") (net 37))
 (segment (start 143.256 48.768) (end 145.288 46.736) (width 0.25) (layer "B.Cu") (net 37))
 (segment (start 143.256 51.816) (end 143.256 48.768) (width 0.25) (layer "B.Cu") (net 37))
 (segment (start 143.002 49.276) (end 145.288 49.276) (width 0.25) (layer "F.Cu") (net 38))
 (segment (start 130.805 57.917) (end 134.361 57.917) (width 0.25) (layer "F.Cu") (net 38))
 (segment (start 134.361 57.917) (end 143.002 49.276) (width 0.25) (layer "F.Cu") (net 38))
 (segment (start 144.267 55.377) (end 145.288 54.356) (width 0.25) (layer "B.Cu") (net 39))
 (segment (start 130.805 55.377) (end 144.267 55.377) (width 0.25) (layer "B.Cu") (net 39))
 (segment (start 129.286 54.356) (end 125.222 54.356) (width 0.25) (layer "F.Cu") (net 40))
 (segment (start 130.805 52.837) (end 129.286 54.356) (width 0.25) (layer "F.Cu") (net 40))
 (via (at 125.222 54.356) (size 0.8) (drill 0.4) (layers "F.Cu" "B.Cu") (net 40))
 (segment (start 130.805 47.493) (end 122.428 39.116) (width 0.25) (layer "B.Cu") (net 40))
 (segment (start 130.805 52.837) (end 130.805 47.493) (width 0.25) (layer "B.Cu") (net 40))
 (segment (start 122.428 92.456) (end 122.428 89.916) (width 0.25) (layer "B.Cu") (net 40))
 (segment (start 125.222 54.356) (end 125.222 87.122) (width 0.25) (layer "B.Cu") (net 40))
 (segment (start 125.222 87.122) (end 122.428 89.916) (width 0.25) (layer "B.Cu") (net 40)))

